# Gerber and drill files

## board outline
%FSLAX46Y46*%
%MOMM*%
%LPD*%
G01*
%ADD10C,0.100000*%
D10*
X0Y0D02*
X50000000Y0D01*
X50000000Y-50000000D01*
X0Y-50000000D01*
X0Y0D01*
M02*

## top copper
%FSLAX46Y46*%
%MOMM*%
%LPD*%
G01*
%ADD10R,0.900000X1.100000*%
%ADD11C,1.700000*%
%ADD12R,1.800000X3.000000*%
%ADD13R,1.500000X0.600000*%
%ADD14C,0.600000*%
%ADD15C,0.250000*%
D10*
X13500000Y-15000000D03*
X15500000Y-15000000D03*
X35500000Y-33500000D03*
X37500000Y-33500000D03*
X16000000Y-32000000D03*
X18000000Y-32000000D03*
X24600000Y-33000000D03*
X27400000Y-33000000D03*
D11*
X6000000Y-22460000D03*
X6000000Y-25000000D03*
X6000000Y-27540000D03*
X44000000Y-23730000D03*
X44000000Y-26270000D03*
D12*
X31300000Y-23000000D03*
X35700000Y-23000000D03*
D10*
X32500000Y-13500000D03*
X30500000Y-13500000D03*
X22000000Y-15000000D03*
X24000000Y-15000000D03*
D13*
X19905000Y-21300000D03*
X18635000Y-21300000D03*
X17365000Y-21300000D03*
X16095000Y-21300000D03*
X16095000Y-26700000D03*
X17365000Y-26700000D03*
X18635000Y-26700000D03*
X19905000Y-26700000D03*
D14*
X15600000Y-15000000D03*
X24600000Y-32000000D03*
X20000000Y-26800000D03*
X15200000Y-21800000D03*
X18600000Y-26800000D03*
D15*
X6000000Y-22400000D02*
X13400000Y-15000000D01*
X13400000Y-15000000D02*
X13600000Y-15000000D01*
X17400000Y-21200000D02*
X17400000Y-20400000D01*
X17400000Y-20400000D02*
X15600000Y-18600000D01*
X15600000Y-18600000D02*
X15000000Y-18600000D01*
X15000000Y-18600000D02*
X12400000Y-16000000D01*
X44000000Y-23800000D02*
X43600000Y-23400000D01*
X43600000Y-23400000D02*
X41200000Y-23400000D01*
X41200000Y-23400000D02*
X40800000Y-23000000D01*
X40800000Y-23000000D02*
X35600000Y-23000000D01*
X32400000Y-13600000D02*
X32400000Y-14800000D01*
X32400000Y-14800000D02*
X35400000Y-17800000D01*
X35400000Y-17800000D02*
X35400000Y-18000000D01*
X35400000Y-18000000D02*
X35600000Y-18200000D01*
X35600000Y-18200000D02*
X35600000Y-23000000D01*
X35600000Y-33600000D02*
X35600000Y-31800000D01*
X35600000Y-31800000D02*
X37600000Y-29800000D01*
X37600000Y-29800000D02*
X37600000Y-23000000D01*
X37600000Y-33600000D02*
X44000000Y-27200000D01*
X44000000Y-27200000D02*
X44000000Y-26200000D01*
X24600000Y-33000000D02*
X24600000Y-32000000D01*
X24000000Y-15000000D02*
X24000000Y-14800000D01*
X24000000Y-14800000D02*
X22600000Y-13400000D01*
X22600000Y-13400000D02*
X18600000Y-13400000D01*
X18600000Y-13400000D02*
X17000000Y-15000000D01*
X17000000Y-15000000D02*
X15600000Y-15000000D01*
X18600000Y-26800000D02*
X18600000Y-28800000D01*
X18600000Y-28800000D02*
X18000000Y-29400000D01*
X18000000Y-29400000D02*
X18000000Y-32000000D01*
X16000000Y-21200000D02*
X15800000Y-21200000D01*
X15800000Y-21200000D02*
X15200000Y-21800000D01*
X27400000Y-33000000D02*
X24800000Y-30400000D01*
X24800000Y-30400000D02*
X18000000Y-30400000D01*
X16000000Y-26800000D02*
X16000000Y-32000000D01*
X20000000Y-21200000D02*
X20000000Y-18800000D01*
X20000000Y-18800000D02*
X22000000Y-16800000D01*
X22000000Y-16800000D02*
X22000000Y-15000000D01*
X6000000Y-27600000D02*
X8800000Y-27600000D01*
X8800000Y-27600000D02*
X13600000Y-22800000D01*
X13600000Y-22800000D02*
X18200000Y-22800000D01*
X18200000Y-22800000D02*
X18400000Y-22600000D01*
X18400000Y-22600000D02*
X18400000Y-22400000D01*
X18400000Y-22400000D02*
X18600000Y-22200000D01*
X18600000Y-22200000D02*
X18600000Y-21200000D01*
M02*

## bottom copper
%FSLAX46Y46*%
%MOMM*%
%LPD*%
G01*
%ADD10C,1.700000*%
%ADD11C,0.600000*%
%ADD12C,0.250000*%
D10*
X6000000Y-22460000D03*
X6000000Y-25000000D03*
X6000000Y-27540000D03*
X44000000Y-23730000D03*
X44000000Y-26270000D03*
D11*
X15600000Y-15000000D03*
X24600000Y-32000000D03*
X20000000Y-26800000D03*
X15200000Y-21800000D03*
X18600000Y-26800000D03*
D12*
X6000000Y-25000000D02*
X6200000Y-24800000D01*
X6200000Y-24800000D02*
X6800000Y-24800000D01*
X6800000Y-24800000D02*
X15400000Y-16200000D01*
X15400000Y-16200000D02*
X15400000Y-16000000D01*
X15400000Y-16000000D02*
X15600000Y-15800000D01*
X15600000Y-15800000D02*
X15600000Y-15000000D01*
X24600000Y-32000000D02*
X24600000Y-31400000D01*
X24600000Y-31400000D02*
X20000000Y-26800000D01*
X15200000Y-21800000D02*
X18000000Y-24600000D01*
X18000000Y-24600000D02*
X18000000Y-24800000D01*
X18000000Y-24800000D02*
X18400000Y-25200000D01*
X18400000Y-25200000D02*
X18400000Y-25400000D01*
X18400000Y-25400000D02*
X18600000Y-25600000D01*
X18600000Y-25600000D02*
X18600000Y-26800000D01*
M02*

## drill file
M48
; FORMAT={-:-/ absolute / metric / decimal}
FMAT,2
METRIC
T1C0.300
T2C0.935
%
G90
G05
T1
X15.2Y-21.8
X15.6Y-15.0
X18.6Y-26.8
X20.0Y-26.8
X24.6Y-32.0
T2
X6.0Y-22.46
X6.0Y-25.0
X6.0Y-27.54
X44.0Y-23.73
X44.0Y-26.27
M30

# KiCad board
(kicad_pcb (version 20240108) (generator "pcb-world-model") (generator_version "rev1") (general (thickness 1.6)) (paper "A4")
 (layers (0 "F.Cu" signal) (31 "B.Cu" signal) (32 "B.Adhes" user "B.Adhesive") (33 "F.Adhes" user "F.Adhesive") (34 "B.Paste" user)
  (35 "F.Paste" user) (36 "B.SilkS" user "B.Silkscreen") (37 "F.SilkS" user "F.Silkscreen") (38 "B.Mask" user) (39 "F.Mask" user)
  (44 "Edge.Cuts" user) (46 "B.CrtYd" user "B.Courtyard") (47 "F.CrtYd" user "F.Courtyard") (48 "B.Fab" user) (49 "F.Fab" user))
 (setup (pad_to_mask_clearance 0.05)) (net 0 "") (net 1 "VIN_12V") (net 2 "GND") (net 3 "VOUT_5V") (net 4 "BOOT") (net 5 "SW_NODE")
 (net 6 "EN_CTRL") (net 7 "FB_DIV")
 (gr_rect (start 0.0 0.0) (end 50.0000 50.0000) (stroke (width 0.1) (type default)) (fill none) (layer "Edge.Cuts"))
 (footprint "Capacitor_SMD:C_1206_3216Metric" (layer "F.Cu") (at 14.5000 15.0000 0)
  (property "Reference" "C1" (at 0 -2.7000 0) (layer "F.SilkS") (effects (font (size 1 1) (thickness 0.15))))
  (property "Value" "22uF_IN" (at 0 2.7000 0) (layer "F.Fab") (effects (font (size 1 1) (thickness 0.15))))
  (pad "1" smd rect (at -1.0000 0.0000) (size 0.9000 1.1000) (layers "F.Cu" "F.Paste" "F.Mask") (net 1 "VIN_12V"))
  (pad "2" smd rect (at 1.0000 0.0000) (size 0.9000 1.1000) (layers "F.Cu" "F.Paste" "F.Mask") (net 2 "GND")))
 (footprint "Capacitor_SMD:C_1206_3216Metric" (layer "F.Cu") (at 36.5000 33.5000 0)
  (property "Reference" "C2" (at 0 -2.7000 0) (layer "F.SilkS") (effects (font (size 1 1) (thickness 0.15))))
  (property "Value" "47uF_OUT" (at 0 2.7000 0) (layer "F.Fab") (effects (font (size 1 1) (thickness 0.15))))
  (pad "1" smd rect (at -1.0000 0.0000) (size 0.9000 1.1000) (layers "F.Cu" "F.Paste" "F.Mask") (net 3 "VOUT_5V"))
  (pad "2" smd rect (at 1.0000 0.0000) (size 0.9000 1.1000) (layers "F.Cu" "F.Paste" "F.Mask") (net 2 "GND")))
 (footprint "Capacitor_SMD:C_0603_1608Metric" (layer "F.Cu") (at 17.0000 32.0000 0)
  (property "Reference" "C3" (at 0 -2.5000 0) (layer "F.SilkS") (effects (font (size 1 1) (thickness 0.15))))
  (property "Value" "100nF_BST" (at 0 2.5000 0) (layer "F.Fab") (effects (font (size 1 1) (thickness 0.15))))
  (pad "1" smd rect (at -1.0000 0.0000) (size 0.9000 1.1000) (layers "F.Cu" "F.Paste" "F.Mask") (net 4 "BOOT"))
  (pad "2" smd rect (at 1.0000 0.0000) (size 0.9000 1.1000) (layers "F.Cu" "F.Paste" "F.Mask") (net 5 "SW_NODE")))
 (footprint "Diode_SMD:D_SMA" (layer "F.Cu") (at 26.0000 33.0000 0)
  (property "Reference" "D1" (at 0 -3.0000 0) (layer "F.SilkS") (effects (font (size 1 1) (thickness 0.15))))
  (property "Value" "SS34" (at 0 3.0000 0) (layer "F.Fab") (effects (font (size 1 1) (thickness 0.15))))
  (pad "1" smd rect (at -1.4000 0.0000) (size 0.9000 1.1000) (layers "F.Cu" "F.Paste" "F.Mask") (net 2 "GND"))
  (pad "2" smd rect (at 1.4000 0.0000) (size 0.9000 1.1000) (layers "F.Cu" "F.Paste" "F.Mask") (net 5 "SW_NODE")))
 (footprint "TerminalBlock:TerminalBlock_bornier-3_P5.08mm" (layer "F.Cu") (at 6.0000 25.0000 0) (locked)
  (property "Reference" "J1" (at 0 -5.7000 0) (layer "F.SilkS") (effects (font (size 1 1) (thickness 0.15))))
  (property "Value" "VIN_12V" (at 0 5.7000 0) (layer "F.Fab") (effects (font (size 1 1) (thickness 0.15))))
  (pad "1" thru_hole circle (at 0.0000 -2.5400) (size 1.7000 1.7000) (drill 0.9350) (layers "*.Cu" "*.Mask") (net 1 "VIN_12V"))
  (pad "2" thru_hole circle (at 0.0000 0.0000) (size 1.7000 1.7000) (drill 0.9350) (layers "*.Cu" "*.Mask") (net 2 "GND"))
  (pad "3" thru_hole circle (at 0.0000 2.5400) (size 1.7000 1.7000) (drill 0.9350) (layers "*.Cu" "*.Mask") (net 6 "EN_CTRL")))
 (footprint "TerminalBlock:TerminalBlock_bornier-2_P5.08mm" (layer "F.Cu") (at 44.0000 25.0000 0) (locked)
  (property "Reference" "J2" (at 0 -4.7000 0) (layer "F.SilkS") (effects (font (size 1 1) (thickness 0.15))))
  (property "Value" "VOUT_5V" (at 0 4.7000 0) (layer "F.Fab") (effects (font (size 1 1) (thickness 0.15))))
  (pad "1" thru_hole circle (at 0.0000 -1.2700) (size 1.7000 1.7000) (drill 0.9350) (layers "*.Cu" "*.Mask") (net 3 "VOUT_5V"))
  (pad "2" thru_hole circle (at 0.0000 1.2700) (size 1.7000 1.7000) (drill 0.9350) (layers "*.Cu" "*.Mask") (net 2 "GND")))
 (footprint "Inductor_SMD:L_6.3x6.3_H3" (layer "F.Cu") (at 33.5000 23.0000 0)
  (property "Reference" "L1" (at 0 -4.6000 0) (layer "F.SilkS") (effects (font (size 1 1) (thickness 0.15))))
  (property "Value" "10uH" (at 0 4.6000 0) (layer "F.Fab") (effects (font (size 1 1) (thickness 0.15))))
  (pad "1" smd rect (at -2.2000 0.0000) (size 1.8000 3.0000) (layers "F.Cu" "F.Paste" "F.Mask") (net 5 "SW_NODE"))
  (pad "2" smd rect (at 2.2000 0.0000) (size 1.8000 3.0000) (layers "F.Cu" "F.Paste" "F.Mask") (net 3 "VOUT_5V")))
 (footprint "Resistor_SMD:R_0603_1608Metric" (layer "F.Cu") (at 31.5000 13.5000 180)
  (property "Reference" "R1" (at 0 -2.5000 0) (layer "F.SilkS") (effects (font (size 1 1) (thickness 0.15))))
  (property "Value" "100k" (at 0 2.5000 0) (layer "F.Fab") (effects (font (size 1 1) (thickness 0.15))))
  (pad "1" smd rect (at -1.0000 0.0000) (size 0.9000 1.1000) (layers "F.Cu" "F.Paste" "F.Mask") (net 3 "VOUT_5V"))
  (pad "2" smd rect (at 1.0000 0.0000) (size 0.9000 1.1000) (layers "F.Cu" "F.Paste" "F.Mask") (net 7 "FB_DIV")))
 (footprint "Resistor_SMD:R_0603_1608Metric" (layer "F.Cu") (at 23.0000 15.0000 0)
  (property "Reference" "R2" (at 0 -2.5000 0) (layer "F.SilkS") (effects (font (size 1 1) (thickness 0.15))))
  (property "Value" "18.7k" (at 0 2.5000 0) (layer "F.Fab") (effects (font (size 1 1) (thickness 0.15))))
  (pad "1" smd rect (at -1.0000 0.0000) (size 0.9000 1.1000) (layers "F.Cu" "F.Paste" "F.Mask") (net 7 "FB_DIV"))
  (pad "2" smd rect (at 1.0000 0.0000) (size 0.9000 1.1000) (layers "F.Cu" "F.Paste" "F.Mask") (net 2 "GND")))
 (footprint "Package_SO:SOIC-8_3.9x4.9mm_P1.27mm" (layer "F.Cu") (at 18.0000 24.0000 270)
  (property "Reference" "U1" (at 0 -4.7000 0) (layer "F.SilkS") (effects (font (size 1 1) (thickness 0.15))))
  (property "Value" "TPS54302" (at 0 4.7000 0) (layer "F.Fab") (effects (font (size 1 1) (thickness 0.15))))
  (pad "1" smd rect (at -2.7000 -1.9050) (size 1.5000 0.6000) (layers "F.Cu" "F.Paste" "F.Mask") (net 4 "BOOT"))
  (pad "2" smd rect (at -2.7000 -0.6350) (size 1.5000 0.6000) (layers "F.Cu" "F.Paste" "F.Mask") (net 1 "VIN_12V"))
  (pad "3" smd rect (at -2.7000 0.6350) (size 1.5000 0.6000) (layers "F.Cu" "F.Paste" "F.Mask") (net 5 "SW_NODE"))
  (pad "4" smd rect (at -2.7000 1.9050) (size 1.5000 0.6000) (layers "F.Cu" "F.Paste" "F.Mask") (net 2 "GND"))
  (pad "5" smd rect (at 2.7000 1.9050) (size 1.5000 0.6000) (layers "F.Cu" "F.Paste" "F.Mask") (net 7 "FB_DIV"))
  (pad "6" smd rect (at 2.7000 0.6350) (size 1.5000 0.6000) (layers "F.Cu" "F.Paste" "F.Mask") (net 6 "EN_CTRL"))
  (pad "7" smd rect (at 2.7000 -0.6350) (size 1.5000 0.6000) (layers "F.Cu" "F.Paste" "F.Mask") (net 1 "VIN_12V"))
  (pad "8" smd rect (at 2.7000 -1.9050) (size 1.5000 0.6000) (layers "F.Cu" "F.Paste" "F.Mask") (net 5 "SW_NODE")))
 (segment (start 6.0000 22.4000) (end 13.4000 15.0000) (width 0.2500) (layer "F.Cu") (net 1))
 (segment (start 13.4000 15.0000) (end 13.6000 15.0000) (width 0.2500) (layer "F.Cu") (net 1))
 (segment (start 17.4000 21.2000) (end 17.4000 20.4000) (width 0.2500) (layer "F.Cu") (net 1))
 (segment (start 17.4000 20.4000) (end 15.6000 18.6000) (width 0.2500) (layer "F.Cu") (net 1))
 (segment (start 15.6000 18.6000) (end 15.0000 18.6000) (width 0.2500) (layer "F.Cu") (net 1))
 (segment (start 15.0000 18.6000) (end 12.4000 16.0000) (width 0.2500) (layer "F.Cu") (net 1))
 (segment (start 44.0000 23.8000) (end 43.6000 23.4000) (width 0.2500) (layer "F.Cu") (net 3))
 (segment (start 43.6000 23.4000) (end 41.2000 23.4000) (width 0.2500) (layer "F.Cu") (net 3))
 (segment (start 41.2000 23.4000) (end 40.8000 23.0000) (width 0.2500) (layer "F.Cu") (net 3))
 (segment (start 40.8000 23.0000) (end 35.6000 23.0000) (width 0.2500) (layer "F.Cu") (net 3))
 (segment (start 32.4000 13.6000) (end 32.4000 14.8000) (width 0.2500) (layer "F.Cu") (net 3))
 (segment (start 32.4000 14.8000) (end 35.4000 17.8000) (width 0.2500) (layer "F.Cu") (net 3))
 (segment (start 35.4000 17.8000) (end 35.4000 18.0000) (width 0.2500) (layer "F.Cu") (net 3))
 (segment (start 35.4000 18.0000) (end 35.6000 18.2000) (width 0.2500) (layer "F.Cu") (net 3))
 (segment (start 35.6000 18.2000) (end 35.6000 23.0000) (width 0.2500) (layer "F.Cu") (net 3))
 (segment (start 35.6000 33.6000) (end 35.6000 31.8000) (width 0.2500) (layer "F.Cu") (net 3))
 (segment (start 35.6000 31.8000) (end 37.6000 29.8000) (width 0.2500) (layer "F.Cu") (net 3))
 (segment (start 37.6000 29.8000) (end 37.6000 23.0000) (width 0.2500) (layer "F.Cu") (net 3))
 (segment (start 6.0000 25.0000) (end 6.2000 24.8000) (width 0.2500) (layer "B.Cu") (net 2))
 (segment (start 6.2000 24.8000) (end 6.8000 24.8000) (width 0.2500) (layer "B.Cu") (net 2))
 (segment (start 6.8000 24.8000) (end 15.4000 16.2000) (width 0.2500) (layer "B.Cu") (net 2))
 (segment (start 15.4000 16.2000) (end 15.4000 16.0000) (width 0.2500) (layer "B.Cu") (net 2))
 (segment (start 15.4000 16.0000) (end 15.6000 15.8000) (width 0.2500) (layer "B.Cu") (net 2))
 (segment (start 15.6000 15.8000) (end 15.6000 15.0000) (width 0.2500) (layer "B.Cu") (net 2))
 (segment (start 37.6000 33.6000) (end 44.0000 27.2000) (width 0.2500) (layer "F.Cu") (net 2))
 (segment (start 44.0000 27.2000) (end 44.0000 26.2000) (width 0.2500) (layer "F.Cu") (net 2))
 (segment (start 24.6000 33.0000) (end 24.6000 32.0000) (width 0.2500) (layer "F.Cu") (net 2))
 (segment (start 24.6000 32.0000) (end 24.6000 31.4000) (width 0.2500) (layer "B.Cu") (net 2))
 (segment (start 24.6000 31.4000) (end 20.0000 26.8000) (width 0.2500) (layer "B.Cu") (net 2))
 (segment (start 24.0000 15.0000) (end 24.0000 14.8000) (width 0.2500) (layer "F.Cu") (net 2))
 (segment (start 24.0000 14.8000) (end 22.6000 13.4000) (width 0.2500) (layer "F.Cu") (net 2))
 (segment (start 22.6000 13.4000) (end 18.6000 13.4000) (width 0.2500) (layer "F.Cu") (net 2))
 (segment (start 18.6000 13.4000) (end 17.0000 15.0000) (width 0.2500) (layer "F.Cu") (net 2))
 (segment (start 17.0000 15.0000) (end 15.6000 15.0000) (width 0.2500) (layer "F.Cu") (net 2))
 (segment (start 18.6000 26.8000) (end 18.6000 28.8000) (width 0.2500) (layer "F.Cu") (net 5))
 (segment (start 18.6000 28.8000) (end 18.0000 29.4000) (width 0.2500) (layer "F.Cu") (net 5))
 (segment (start 18.0000 29.4000) (end 18.0000 32.0000) (width 0.2500) (layer "F.Cu") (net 5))
 (segment (start 16.0000 21.2000) (end 15.8000 21.2000) (width 0.2500) (layer "F.Cu") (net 5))
 (segment (start 15.8000 21.2000) (end 15.2000 21.8000) (width 0.2500) (layer "F.Cu") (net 5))
 (segment (start 15.2000 21.8000) (end 18.0000 24.6000) (width 0.2500) (layer "B.Cu") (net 5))
 (segment (start 18.0000 24.6000) (end 18.0000 24.8000) (width 0.2500) (layer "B.Cu") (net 5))
 (segment (start 18.0000 24.8000) (end 18.4000 25.2000) (width 0.2500) (layer "B.Cu") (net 5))
 (segment (start 18.4000 25.2000) (end 18.4000 25.4000) (width 0.2500) (layer "B.Cu") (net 5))
 (segment (start 18.4000 25.4000) (end 18.6000 25.6000) (width 0.2500) (layer "B.Cu") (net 5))
 (segment (start 18.6000 25.6000) (end 18.6000 26.8000) (width 0.2500) (layer "B.Cu") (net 5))
 (segment (start 27.4000 33.0000) (end 24.8000 30.4000) (width 0.2500) (layer "F.Cu") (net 5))
 (segment (start 24.8000 30.4000) (end 18.0000 30.4000) (width 0.2500) (layer "F.Cu") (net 5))
 (segment (start 16.0000 26.8000) (end 16.0000 32.0000) (width 0.2500) (layer "F.Cu") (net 4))
 (segment (start 20.0000 21.2000) (end 20.0000 18.8000) (width 0.2500) (layer "F.Cu") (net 7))
 (segment (start 20.0000 18.8000) (end 22.0000 16.8000) (width 0.2500) (layer "F.Cu") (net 7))
 (segment (start 22.0000 16.8000) (end 22.0000 15.0000) (width 0.2500) (layer "F.Cu") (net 7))
 (segment (start 6.0000 27.6000) (end 8.8000 27.6000) (width 0.2500) (layer "F.Cu") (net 6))
 (segment (start 8.8000 27.6000) (end 13.6000 22.8000) (width 0.2500) (layer "F.Cu") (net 6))
 (segment (start 13.6000 22.8000) (end 18.2000 22.8000) (width 0.2500) (layer "F.Cu") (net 6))
 (segment (start 18.2000 22.8000) (end 18.4000 22.6000) (width 0.2500) (layer "F.Cu") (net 6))
 (segment (start 18.4000 22.6000) (end 18.4000 22.4000) (width 0.2500) (layer "F.Cu") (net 6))
 (segment (start 18.4000 22.4000) (end 18.6000 22.2000) (width 0.2500) (layer "F.Cu") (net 6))
 (segment (start 18.6000 22.2000) (end 18.6000 21.2000) (width 0.2500) (layer "F.Cu") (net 6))
 (via (at 15.6000 15.0000) (size 0.6000) (drill 0.3000) (layers "F.Cu" "B.Cu") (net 2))
 (via (at 24.6000 32.0000) (size 0.6000) (drill 0.3000) (layers "F.Cu" "B.Cu") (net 2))
 (via (at 20.0000 26.8000) (size 0.6000) (drill 0.3000) (layers "F.Cu" "B.Cu") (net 2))
 (via (at 15.2000 21.8000) (size 0.6000) (drill 0.3000) (layers "F.Cu" "B.Cu") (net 5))
 (via (at 18.6000 26.8000) (size 0.6000) (drill 0.3000) (layers "F.Cu" "B.Cu") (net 5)))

